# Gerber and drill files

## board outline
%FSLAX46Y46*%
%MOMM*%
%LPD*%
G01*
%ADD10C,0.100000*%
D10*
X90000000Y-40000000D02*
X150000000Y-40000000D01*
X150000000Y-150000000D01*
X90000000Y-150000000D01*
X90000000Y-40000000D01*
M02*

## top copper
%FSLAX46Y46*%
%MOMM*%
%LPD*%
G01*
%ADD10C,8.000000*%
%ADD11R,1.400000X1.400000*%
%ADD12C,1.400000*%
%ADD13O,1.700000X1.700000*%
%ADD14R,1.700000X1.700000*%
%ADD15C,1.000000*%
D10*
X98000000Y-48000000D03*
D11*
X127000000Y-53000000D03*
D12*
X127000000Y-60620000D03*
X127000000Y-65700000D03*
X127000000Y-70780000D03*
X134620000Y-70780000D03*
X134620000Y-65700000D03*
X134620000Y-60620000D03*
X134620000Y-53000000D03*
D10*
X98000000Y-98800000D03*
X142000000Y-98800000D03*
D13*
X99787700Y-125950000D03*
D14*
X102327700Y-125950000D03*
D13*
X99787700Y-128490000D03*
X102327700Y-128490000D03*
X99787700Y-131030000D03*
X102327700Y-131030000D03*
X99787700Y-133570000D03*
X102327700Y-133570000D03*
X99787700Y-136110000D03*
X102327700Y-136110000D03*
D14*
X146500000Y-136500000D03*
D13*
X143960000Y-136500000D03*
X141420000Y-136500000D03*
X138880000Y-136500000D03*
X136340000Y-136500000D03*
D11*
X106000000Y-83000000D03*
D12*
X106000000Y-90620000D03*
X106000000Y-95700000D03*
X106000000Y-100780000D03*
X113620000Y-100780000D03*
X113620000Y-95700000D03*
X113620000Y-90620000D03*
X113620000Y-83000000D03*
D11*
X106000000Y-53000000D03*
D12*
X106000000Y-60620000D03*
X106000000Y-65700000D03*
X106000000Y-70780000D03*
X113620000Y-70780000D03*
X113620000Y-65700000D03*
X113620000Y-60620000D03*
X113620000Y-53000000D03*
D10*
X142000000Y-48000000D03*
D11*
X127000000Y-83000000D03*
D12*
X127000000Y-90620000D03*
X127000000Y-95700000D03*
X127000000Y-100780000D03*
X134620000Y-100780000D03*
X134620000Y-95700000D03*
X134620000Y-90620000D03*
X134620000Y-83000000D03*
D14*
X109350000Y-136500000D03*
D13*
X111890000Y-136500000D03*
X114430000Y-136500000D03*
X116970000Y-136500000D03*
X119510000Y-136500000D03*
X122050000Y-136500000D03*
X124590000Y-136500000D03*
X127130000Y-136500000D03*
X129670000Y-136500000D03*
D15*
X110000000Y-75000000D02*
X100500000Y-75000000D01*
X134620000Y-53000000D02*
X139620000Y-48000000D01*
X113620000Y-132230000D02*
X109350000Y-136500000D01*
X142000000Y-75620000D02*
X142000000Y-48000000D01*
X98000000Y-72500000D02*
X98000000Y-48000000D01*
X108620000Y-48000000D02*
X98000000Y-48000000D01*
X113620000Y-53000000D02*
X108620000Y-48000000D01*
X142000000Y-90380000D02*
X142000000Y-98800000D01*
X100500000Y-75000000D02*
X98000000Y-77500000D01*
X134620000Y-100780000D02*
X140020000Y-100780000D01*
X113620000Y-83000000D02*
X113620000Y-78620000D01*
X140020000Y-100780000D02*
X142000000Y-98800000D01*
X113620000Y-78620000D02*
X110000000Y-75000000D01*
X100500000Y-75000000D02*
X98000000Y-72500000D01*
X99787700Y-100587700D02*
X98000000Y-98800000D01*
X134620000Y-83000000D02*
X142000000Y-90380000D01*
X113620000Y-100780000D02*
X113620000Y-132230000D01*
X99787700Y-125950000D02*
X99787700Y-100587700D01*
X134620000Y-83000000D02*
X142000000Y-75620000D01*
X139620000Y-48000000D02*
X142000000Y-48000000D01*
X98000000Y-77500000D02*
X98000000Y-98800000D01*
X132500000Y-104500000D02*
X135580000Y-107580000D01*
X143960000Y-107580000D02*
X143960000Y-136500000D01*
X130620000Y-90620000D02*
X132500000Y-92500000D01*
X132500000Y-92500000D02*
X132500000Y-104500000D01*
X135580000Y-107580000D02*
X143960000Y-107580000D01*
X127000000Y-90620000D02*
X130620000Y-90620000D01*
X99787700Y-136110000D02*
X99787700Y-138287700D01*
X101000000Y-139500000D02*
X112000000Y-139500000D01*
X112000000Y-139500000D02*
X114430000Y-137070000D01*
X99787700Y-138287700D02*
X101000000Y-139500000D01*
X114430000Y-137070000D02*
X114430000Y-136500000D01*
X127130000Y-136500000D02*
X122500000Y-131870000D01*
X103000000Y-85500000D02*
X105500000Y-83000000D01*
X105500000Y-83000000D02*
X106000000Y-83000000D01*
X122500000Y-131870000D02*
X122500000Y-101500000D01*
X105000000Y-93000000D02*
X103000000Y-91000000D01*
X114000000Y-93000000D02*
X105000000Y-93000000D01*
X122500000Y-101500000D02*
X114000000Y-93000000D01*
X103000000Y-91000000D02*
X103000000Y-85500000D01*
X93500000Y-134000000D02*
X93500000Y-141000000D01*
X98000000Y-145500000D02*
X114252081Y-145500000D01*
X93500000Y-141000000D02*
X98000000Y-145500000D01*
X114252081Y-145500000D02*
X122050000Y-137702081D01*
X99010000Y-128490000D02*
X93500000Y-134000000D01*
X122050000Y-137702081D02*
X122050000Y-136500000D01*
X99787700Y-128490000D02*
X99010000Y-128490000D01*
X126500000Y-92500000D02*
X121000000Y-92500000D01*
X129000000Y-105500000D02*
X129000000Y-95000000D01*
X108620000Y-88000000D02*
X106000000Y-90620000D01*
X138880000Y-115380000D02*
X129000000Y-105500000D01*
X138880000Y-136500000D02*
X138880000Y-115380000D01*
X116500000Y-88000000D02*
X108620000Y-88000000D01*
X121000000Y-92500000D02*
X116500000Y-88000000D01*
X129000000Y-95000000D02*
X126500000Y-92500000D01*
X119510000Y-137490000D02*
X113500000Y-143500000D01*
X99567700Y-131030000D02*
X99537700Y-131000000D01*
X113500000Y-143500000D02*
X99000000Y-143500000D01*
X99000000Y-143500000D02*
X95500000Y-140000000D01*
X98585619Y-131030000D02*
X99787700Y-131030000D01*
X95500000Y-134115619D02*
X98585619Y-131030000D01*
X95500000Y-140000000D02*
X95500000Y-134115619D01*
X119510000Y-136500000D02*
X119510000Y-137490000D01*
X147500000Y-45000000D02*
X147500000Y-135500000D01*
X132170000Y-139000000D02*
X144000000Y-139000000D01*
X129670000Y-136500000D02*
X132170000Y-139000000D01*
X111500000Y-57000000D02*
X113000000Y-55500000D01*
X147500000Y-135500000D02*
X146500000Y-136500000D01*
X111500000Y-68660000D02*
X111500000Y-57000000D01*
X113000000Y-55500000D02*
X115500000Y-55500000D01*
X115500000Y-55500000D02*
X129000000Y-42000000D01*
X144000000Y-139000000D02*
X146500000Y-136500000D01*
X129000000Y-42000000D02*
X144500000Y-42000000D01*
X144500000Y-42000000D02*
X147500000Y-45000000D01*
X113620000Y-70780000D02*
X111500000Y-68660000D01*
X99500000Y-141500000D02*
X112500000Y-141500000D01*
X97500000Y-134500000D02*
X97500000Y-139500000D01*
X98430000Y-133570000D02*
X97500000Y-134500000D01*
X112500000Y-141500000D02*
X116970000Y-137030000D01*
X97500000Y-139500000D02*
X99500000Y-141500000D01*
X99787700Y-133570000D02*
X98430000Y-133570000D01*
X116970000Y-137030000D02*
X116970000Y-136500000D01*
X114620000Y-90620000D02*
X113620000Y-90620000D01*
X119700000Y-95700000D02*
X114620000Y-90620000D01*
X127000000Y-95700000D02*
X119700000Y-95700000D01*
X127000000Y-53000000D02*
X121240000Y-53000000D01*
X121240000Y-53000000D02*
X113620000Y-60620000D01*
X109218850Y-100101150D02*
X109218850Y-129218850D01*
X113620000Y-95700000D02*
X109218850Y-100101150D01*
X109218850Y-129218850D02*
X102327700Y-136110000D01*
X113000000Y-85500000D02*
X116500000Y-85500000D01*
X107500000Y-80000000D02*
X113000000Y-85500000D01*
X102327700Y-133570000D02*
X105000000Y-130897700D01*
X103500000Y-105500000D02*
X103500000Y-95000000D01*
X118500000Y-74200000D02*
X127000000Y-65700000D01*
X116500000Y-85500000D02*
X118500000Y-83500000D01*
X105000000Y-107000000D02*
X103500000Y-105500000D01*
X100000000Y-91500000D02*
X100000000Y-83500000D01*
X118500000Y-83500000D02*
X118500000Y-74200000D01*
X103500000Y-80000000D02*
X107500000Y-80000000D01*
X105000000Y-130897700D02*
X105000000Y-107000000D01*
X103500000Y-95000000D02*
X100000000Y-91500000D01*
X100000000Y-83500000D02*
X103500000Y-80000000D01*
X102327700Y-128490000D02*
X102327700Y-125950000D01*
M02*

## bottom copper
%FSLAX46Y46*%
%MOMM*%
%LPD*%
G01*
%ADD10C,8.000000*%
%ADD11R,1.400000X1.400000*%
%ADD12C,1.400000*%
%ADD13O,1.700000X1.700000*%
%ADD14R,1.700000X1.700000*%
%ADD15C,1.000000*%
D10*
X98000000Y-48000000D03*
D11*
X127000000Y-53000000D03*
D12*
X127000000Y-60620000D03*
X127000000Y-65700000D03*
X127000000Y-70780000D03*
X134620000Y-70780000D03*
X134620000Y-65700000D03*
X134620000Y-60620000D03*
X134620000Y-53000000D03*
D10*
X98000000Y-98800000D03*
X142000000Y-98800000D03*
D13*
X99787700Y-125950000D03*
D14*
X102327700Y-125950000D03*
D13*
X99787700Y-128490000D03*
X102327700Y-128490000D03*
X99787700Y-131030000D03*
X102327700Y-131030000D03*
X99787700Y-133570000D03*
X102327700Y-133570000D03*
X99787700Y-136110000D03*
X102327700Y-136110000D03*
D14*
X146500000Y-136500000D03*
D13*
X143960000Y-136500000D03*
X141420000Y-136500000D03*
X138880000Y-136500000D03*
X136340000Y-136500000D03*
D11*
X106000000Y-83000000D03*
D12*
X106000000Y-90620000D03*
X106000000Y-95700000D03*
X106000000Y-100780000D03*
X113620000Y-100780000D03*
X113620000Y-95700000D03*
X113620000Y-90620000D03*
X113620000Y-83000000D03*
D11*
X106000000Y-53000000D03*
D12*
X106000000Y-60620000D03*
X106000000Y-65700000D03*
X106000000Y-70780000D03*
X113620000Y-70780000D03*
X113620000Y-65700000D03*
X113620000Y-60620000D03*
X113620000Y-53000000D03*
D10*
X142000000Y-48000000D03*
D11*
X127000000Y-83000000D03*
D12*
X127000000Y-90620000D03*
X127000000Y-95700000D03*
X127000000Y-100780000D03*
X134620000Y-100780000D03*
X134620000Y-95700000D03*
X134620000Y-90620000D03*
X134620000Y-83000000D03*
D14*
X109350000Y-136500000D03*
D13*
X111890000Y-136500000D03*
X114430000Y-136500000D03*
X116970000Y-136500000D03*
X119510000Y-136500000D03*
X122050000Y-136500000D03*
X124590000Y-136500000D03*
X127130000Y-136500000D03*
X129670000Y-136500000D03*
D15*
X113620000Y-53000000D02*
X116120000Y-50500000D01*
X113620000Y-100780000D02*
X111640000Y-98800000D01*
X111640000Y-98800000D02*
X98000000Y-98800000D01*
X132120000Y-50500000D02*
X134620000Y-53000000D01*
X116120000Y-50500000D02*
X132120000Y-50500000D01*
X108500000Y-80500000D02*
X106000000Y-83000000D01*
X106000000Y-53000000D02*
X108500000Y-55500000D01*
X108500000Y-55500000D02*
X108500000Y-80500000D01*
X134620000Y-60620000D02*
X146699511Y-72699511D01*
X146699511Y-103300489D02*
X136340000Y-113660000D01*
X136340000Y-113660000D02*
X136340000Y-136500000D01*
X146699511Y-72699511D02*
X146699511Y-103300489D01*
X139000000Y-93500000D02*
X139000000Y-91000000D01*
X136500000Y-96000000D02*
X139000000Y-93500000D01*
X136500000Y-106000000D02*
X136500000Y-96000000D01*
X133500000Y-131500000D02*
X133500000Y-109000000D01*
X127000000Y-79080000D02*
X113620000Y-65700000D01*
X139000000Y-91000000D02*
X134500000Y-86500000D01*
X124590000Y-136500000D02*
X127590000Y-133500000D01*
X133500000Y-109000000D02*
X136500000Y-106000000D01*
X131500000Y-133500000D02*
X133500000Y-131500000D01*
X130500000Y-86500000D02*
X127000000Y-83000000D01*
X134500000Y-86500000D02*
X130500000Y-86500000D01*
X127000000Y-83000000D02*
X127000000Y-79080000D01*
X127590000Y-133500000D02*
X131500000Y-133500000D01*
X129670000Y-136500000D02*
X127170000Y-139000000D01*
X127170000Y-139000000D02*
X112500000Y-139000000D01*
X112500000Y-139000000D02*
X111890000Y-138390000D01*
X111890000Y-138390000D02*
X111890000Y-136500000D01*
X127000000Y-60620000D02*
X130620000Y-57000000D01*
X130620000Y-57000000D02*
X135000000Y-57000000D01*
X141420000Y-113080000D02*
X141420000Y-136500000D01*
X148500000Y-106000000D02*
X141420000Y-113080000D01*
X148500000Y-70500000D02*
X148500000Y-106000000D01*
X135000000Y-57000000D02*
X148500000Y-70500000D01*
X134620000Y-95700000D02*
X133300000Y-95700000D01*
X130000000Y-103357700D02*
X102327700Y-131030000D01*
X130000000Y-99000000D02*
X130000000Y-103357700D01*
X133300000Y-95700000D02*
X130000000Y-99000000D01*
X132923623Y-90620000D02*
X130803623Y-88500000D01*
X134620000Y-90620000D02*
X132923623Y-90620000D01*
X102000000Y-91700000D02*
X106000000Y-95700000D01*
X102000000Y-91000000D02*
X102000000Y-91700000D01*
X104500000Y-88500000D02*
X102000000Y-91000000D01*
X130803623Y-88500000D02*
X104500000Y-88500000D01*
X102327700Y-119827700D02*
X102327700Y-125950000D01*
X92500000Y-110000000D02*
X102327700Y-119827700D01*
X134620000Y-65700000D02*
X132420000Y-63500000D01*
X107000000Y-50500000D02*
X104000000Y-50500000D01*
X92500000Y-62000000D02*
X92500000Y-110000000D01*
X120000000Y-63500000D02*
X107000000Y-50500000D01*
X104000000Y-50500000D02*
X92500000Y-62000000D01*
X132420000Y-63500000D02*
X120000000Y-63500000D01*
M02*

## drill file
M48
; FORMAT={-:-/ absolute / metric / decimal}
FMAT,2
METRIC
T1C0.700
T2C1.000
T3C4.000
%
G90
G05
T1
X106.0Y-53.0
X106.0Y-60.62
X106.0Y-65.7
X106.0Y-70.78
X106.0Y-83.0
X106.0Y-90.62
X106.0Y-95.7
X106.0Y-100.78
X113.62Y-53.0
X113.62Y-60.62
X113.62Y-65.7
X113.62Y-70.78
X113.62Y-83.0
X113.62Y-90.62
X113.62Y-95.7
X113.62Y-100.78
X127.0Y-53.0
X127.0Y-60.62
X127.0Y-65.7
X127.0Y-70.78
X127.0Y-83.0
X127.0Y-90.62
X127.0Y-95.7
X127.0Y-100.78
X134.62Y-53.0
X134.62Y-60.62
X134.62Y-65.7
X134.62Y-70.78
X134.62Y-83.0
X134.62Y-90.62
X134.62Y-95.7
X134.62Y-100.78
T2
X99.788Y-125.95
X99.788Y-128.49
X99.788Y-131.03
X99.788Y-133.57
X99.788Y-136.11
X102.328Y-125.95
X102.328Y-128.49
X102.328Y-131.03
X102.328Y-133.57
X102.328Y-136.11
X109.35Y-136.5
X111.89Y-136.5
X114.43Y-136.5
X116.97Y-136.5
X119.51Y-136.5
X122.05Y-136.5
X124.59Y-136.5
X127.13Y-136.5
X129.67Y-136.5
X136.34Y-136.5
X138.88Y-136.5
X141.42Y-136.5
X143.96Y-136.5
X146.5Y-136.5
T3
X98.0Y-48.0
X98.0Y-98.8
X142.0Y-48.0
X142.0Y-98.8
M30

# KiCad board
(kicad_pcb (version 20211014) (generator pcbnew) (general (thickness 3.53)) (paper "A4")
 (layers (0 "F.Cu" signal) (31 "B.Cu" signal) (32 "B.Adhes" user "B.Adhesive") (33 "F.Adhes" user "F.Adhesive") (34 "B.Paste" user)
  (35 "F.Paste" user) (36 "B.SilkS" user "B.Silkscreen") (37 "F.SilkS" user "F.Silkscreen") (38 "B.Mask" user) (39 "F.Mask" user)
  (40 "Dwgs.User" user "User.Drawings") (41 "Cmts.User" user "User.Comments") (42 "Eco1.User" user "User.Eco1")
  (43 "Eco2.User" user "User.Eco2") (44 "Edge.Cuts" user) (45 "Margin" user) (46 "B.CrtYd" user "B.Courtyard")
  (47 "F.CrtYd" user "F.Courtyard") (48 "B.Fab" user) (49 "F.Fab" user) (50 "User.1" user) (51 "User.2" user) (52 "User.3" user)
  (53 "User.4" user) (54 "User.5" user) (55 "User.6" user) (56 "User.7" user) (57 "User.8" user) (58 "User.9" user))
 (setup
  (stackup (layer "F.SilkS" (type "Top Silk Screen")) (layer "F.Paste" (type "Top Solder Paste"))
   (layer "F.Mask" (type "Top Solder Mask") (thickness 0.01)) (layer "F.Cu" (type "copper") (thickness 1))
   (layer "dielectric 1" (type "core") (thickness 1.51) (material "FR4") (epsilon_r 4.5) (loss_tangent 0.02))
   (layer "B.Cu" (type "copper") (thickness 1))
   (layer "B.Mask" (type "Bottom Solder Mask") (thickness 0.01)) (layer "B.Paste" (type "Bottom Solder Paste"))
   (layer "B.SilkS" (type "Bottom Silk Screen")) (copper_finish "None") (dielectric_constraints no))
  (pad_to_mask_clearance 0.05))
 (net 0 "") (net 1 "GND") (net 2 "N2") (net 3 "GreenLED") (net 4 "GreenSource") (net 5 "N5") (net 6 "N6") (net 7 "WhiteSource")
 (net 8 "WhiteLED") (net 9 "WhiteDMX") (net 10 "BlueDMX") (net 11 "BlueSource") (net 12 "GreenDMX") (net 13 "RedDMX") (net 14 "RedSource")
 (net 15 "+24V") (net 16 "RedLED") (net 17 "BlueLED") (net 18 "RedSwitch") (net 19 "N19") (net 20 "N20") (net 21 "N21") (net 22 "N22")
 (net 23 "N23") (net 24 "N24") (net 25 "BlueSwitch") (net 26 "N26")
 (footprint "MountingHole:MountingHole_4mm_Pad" (layer "F.Cu") (at 98 48)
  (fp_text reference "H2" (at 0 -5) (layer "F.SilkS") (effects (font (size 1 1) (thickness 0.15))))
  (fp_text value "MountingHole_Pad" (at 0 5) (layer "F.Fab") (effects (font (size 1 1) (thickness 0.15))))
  (pad "1" thru_hole circle (at 0 0) (size 8 8) (drill 4) (layers *.Cu *.Mask) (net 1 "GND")))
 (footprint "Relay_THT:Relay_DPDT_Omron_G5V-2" (layer "F.Cu") (at 127 53)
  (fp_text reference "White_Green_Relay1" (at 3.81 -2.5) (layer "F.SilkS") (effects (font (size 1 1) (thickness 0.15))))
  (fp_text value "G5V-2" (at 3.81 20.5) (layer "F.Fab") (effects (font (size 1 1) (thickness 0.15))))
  (pad "1" thru_hole rect (at 0 0) (size 1.4 1.4) (drill 0.7) (layers *.Cu *.Mask) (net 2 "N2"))
  (pad "4" thru_hole circle (at 0 7.62) (size 1.4 1.4) (drill 0.7) (layers *.Cu *.Mask) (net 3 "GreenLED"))
  (pad "6" thru_hole circle (at 0 12.7) (size 1.4 1.4) (drill 0.7) (layers *.Cu *.Mask) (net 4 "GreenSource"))
  (pad "8" thru_hole circle (at 0 17.78) (size 1.4 1.4) (drill 0.7) (layers *.Cu *.Mask) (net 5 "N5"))
  (pad "9" thru_hole circle (at 7.62 17.78) (size 1.4 1.4) (drill 0.7) (layers *.Cu *.Mask) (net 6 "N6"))
  (pad "11" thru_hole circle (at 7.62 12.7) (size 1.4 1.4) (drill 0.7) (layers *.Cu *.Mask) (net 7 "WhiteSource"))
  (pad "13" thru_hole circle (at 7.62 7.62) (size 1.4 1.4) (drill 0.7) (layers *.Cu *.Mask) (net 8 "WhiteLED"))
  (pad "16" thru_hole circle (at 7.62 0) (size 1.4 1.4) (drill 0.7) (layers *.Cu *.Mask) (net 1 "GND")))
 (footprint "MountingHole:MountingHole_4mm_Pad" (layer "F.Cu") (at 98 98.8)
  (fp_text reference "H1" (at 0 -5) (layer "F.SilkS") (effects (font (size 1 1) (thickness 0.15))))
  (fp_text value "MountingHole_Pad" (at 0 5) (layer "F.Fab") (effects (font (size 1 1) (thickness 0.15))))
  (pad "1" thru_hole circle (at 0 0) (size 8 8) (drill 4) (layers *.Cu *.Mask) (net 1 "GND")))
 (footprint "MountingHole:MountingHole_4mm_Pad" (layer "F.Cu") (at 142 98.8)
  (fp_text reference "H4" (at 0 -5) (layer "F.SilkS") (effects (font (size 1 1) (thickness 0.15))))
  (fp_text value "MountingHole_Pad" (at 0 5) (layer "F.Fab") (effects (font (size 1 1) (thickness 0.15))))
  (pad "1" thru_hole circle (at 0 0) (size 8 8) (drill 4) (layers *.Cu *.Mask) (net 1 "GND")))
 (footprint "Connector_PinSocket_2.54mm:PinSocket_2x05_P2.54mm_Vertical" (layer "F.Cu") (at 102.3277 125.95)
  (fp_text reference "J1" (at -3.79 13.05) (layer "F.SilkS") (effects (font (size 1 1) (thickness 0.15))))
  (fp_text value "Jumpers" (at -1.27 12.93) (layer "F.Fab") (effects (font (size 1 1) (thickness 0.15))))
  (pad "1a" thru_hole oval (at -2.54 0) (size 1.7 1.7) (drill 1) (layers *.Cu *.Mask) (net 1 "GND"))
  (pad "1b" thru_hole rect (at 0 0) (size 1.7 1.7) (drill 1) (layers *.Cu *.Mask) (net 7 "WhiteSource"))
  (pad "2a" thru_hole oval (at -2.54 2.54) (size 1.7 1.7) (drill 1) (layers *.Cu *.Mask) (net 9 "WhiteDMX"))
  (pad "2b" thru_hole oval (at 0 2.54) (size 1.7 1.7) (drill 1) (layers *.Cu *.Mask) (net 7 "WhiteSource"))
  (pad "3a" thru_hole oval (at -2.54 5.08) (size 1.7 1.7) (drill 1) (layers *.Cu *.Mask) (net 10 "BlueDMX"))
  (pad "3b" thru_hole oval (at 0 5.08) (size 1.7 1.7) (drill 1) (layers *.Cu *.Mask) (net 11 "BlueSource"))
  (pad "4a" thru_hole oval (at -2.54 7.62) (size 1.7 1.7) (drill 1) (layers *.Cu *.Mask) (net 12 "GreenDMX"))
  (pad "4b" thru_hole oval (at 0 7.62) (size 1.7 1.7) (drill 1) (layers *.Cu *.Mask) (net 4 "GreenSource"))
  (pad "5a" thru_hole oval (at -2.54 10.16) (size 1.7 1.7) (drill 1) (layers *.Cu *.Mask) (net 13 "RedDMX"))
  (pad "5b" thru_hole oval (at 0 10.16) (size 1.7 1.7) (drill 1) (layers *.Cu *.Mask) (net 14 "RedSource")))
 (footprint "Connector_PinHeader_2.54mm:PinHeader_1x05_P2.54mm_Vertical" (layer "F.Cu") (at 146.5 136.5 -90)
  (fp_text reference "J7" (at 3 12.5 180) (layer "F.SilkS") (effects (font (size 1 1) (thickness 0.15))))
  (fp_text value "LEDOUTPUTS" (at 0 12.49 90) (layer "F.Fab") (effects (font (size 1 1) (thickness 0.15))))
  (pad "1" thru_hole rect (at 0 0 270) (size 1.7 1.7) (drill 1) (layers *.Cu *.Mask) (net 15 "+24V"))
  (pad "2" thru_hole oval (at 0 2.54 270) (size 1.7 1.7) (drill 1) (layers *.Cu *.Mask) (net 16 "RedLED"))
  (pad "3" thru_hole oval (at 0 5.08 270) (size 1.7 1.7) (drill 1) (layers *.Cu *.Mask) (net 3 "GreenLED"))
  (pad "4" thru_hole oval (at 0 7.62 270) (size 1.7 1.7) (drill 1) (layers *.Cu *.Mask) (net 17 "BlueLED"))
  (pad "5" thru_hole oval (at 0 10.16 270) (size 1.7 1.7) (drill 1) (layers *.Cu *.Mask) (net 8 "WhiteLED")))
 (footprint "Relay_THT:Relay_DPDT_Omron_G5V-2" (layer "F.Cu") (at 106 83)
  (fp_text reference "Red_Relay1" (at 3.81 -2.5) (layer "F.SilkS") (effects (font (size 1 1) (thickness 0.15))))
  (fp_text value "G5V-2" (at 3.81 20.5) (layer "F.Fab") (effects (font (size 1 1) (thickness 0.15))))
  (pad "1" thru_hole rect (at 0 0) (size 1.4 1.4) (drill 0.7) (layers *.Cu *.Mask) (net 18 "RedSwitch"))
  (pad "4" thru_hole circle (at 0 7.62) (size 1.4 1.4) (drill 0.7) (layers *.Cu *.Mask) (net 17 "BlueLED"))
  (pad "6" thru_hole circle (at 0 12.7) (size 1.4 1.4) (drill 0.7) (layers *.Cu *.Mask) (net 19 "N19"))
  (pad "8" thru_hole circle (at 0 17.78) (size 1.4 1.4) (drill 0.7) (layers *.Cu *.Mask) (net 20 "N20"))
  (pad "9" thru_hole circle (at 7.62 17.78) (size 1.4 1.4) (drill 0.7) (layers *.Cu *.Mask) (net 1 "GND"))
  (pad "11" thru_hole circle (at 7.62 12.7) (size 1.4 1.4) (drill 0.7) (layers *.Cu *.Mask) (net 14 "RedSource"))
  (pad "13" thru_hole circle (at 7.62 7.62) (size 1.4 1.4) (drill 0.7) (layers *.Cu *.Mask) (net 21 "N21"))
  (pad "16" thru_hole circle (at 7.62 0) (size 1.4 1.4) (drill 0.7) (layers *.Cu *.Mask) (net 1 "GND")))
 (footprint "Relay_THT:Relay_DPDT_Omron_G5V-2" (layer "F.Cu") (at 106 53)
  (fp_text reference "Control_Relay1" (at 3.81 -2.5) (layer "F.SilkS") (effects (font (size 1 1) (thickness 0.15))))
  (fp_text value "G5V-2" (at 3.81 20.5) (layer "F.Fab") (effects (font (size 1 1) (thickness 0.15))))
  (pad "1" thru_hole rect (at 0 0) (size 1.4 1.4) (drill 0.7) (layers *.Cu *.Mask) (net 18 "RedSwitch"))
  (pad "4" thru_hole circle (at 0 7.62) (size 1.4 1.4) (drill 0.7) (layers *.Cu *.Mask) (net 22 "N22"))
  (pad "6" thru_hole circle (at 0 12.7) (size 1.4 1.4) (drill 0.7) (layers *.Cu *.Mask) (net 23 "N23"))
  (pad "8" thru_hole circle (at 0 17.78) (size 1.4 1.4) (drill 0.7) (layers *.Cu *.Mask) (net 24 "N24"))
  (pad "9" thru_hole circle (at 7.62 17.78) (size 1.4 1.4) (drill 0.7) (layers *.Cu *.Mask) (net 15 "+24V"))
  (pad "11" thru_hole circle (at 7.62 12.7) (size 1.4 1.4) (drill 0.7) (layers *.Cu *.Mask) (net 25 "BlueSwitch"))
  (pad "13" thru_hole circle (at 7.62 7.62) (size 1.4 1.4) (drill 0.7) (layers *.Cu *.Mask) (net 2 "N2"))
  (pad "16" thru_hole circle (at 7.62 0) (size 1.4 1.4) (drill 0.7) (layers *.Cu *.Mask) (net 1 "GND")))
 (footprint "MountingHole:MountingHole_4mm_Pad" (layer "F.Cu") (at 142 48)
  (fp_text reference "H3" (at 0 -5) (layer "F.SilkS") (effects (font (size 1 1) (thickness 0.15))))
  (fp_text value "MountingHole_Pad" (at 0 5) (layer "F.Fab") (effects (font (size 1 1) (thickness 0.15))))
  (pad "1" thru_hole circle (at 0 0) (size 8 8) (drill 4) (layers *.Cu *.Mask) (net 1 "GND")))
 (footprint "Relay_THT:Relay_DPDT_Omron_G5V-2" (layer "F.Cu") (at 127 83)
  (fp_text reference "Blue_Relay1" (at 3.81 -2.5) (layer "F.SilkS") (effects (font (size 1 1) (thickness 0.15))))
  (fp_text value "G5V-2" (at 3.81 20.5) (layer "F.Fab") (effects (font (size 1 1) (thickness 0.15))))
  (pad "1" thru_hole rect (at 0 0) (size 1.4 1.4) (drill 0.7) (layers *.Cu *.Mask) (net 25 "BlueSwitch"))
  (pad "4" thru_hole circle (at 0 7.62) (size 1.4 1.4) (drill 0.7) (layers *.Cu *.Mask) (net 16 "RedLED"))
  (pad "6" thru_hole circle (at 0 12.7) (size 1.4 1.4) (drill 0.7) (layers *.Cu *.Mask) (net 21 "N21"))
  (pad "8" thru_hole circle (at 0 17.78) (size 1.4 1.4) (drill 0.7) (layers *.Cu *.Mask) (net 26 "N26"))
  (pad "9" thru_hole circle (at 7.62 17.78) (size 1.4 1.4) (drill 0.7) (layers *.Cu *.Mask) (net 1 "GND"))
  (pad "11" thru_hole circle (at 7.62 12.7) (size 1.4 1.4) (drill 0.7) (layers *.Cu *.Mask) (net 11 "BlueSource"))
  (pad "13" thru_hole circle (at 7.62 7.62) (size 1.4 1.4) (drill 0.7) (layers *.Cu *.Mask) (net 19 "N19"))
  (pad "16" thru_hole circle (at 7.62 0) (size 1.4 1.4) (drill 0.7) (layers *.Cu *.Mask) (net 1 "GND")))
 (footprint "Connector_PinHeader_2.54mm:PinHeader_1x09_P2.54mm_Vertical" (layer "F.Cu") (at 109.35 136.5 90)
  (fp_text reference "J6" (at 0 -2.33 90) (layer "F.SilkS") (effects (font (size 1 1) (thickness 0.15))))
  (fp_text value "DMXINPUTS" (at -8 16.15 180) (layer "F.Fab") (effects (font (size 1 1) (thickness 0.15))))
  (pad "1" thru_hole rect (at 0 0 90) (size 1.7 1.7) (drill 1) (layers *.Cu *.Mask) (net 1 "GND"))
  (pad "2" thru_hole oval (at 0 2.54 90) (size 1.7 1.7) (drill 1) (layers *.Cu *.Mask) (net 15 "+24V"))
  (pad "3" thru_hole oval (at 0 5.08 90) (size 1.7 1.7) (drill 1) (layers *.Cu *.Mask) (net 13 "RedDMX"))
  (pad "4" thru_hole oval (at 0 7.62 90) (size 1.7 1.7) (drill 1) (layers *.Cu *.Mask) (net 12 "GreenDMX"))
  (pad "5" thru_hole oval (at 0 10.16 90) (size 1.7 1.7) (drill 1) (layers *.Cu *.Mask) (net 10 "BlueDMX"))
  (pad "6" thru_hole oval (at 0 12.7 90) (size 1.7 1.7) (drill 1) (layers *.Cu *.Mask) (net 9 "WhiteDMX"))
  (pad "7" thru_hole oval (at 0 15.24 90) (size 1.7 1.7) (drill 1) (layers *.Cu *.Mask) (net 25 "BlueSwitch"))
  (pad "8" thru_hole oval (at 0 17.78 90) (size 1.7 1.7) (drill 1) (layers *.Cu *.Mask) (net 18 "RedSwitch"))
  (pad "9" thru_hole oval (at 0 20.32 90) (size 1.7 1.7) (drill 1) (layers *.Cu *.Mask) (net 15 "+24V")))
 (gr_rect (start 90 40) (end 150 150) (layer "Edge.Cuts") (width 0.1) (fill none))
 (segment (start 110 75) (end 100.5 75) (width 1) (layer "F.Cu") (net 1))
 (segment (start 134.62 53) (end 139.62 48) (width 1) (layer "F.Cu") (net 1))
 (segment (start 113.62 132.23) (end 109.35 136.5) (width 1) (layer "F.Cu") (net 1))
 (segment (start 142 75.62) (end 142 48) (width 1) (layer "F.Cu") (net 1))
 (segment (start 98 72.5) (end 98 48) (width 1) (layer "F.Cu") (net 1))
 (segment (start 108.62 48) (end 98 48) (width 1) (layer "F.Cu") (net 1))
 (segment (start 113.62 53) (end 108.62 48) (width 1) (layer "F.Cu") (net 1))
 (segment (start 142 90.38) (end 142 98.8) (width 1) (layer "F.Cu") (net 1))
 (segment (start 100.5 75) (end 98 77.5) (width 1) (layer "F.Cu") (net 1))
 (segment (start 134.62 100.78) (end 140.02 100.78) (width 1) (layer "F.Cu") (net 1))
 (segment (start 113.62 83) (end 113.62 78.62) (width 1) (layer "F.Cu") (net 1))
 (segment (start 140.02 100.78) (end 142 98.8) (width 1) (layer "F.Cu") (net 1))
 (segment (start 113.62 78.62) (end 110 75) (width 1) (layer "F.Cu") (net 1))
 (segment (start 100.5 75) (end 98 72.5) (width 1) (layer "F.Cu") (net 1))
 (segment (start 99.7877 100.5877) (end 98 98.8) (width 1) (layer "F.Cu") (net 1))
 (segment (start 134.62 83) (end 142 90.38) (width 1) (layer "F.Cu") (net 1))
 (segment (start 113.62 100.78) (end 113.62 132.23) (width 1) (layer "F.Cu") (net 1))
 (segment (start 99.7877 125.95) (end 99.7877 100.5877) (width 1) (layer "F.Cu") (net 1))
 (segment (start 134.62 83) (end 142 75.62) (width 1) (layer "F.Cu") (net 1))
 (segment (start 139.62 48) (end 142 48) (width 1) (layer "F.Cu") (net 1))
 (segment (start 98 77.5) (end 98 98.8) (width 1) (layer "F.Cu") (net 1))
 (segment (start 113.62 53) (end 116.12 50.5) (width 1) (layer "B.Cu") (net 1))
 (segment (start 113.62 100.78) (end 111.64 98.8) (width 1) (layer "B.Cu") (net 1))
 (segment (start 111.64 98.8) (end 98 98.8) (width 1) (layer "B.Cu") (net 1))
 (segment (start 132.12 50.5) (end 134.62 53) (width 1) (layer "B.Cu") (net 1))
 (segment (start 116.12 50.5) (end 132.12 50.5) (width 1) (layer "B.Cu") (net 1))
 (segment (start 132.5 104.5) (end 135.58 107.58) (width 1) (layer "F.Cu") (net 16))
 (segment (start 143.96 107.58) (end 143.96 136.5) (width 1) (layer "F.Cu") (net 16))
 (segment (start 130.62 90.62) (end 132.5 92.5) (width 1) (layer "F.Cu") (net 16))
 (segment (start 132.5 92.5) (end 132.5 104.5) (width 1) (layer "F.Cu") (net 16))
 (segment (start 135.58 107.58) (end 143.96 107.58) (width 1) (layer "F.Cu") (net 16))
 (segment (start 127 90.62) (end 130.62 90.62) (width 1) (layer "F.Cu") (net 16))
 (segment (start 99.7877 136.11) (end 99.7877 138.2877) (width 1) (layer "F.Cu") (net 13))
 (segment (start 101 139.5) (end 112 139.5) (width 1) (layer "F.Cu") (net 13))
 (segment (start 112 139.5) (end 114.43 137.07) (width 1) (layer "F.Cu") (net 13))
 (segment (start 99.7877 138.2877) (end 101 139.5) (width 1) (layer "F.Cu") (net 13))
 (segment (start 114.43 137.07) (end 114.43 136.5) (width 1) (layer "F.Cu") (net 13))
 (segment (start 127.13 136.5) (end 122.5 131.87) (width 1) (layer "F.Cu") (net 18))
 (segment (start 103 85.5) (end 105.5 83) (width 1) (layer "F.Cu") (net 18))
 (segment (start 105.5 83) (end 106 83) (width 1) (layer "F.Cu") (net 18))
 (segment (start 122.5 131.87) (end 122.5 101.5) (width 1) (layer "F.Cu") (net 18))
 (segment (start 105 93) (end 103 91) (width 1) (layer "F.Cu") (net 18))
 (segment (start 114 93) (end 105 93) (width 1) (layer "F.Cu") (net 18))
 (segment (start 122.5 101.5) (end 114 93) (width 1) (layer "F.Cu") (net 18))
 (segment (start 103 91) (end 103 85.5) (width 1) (layer "F.Cu") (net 18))
 (segment (start 108.5 80.5) (end 106 83) (width 1) (layer "B.Cu") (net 18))
 (segment (start 106 53) (end 108.5 55.5) (width 1) (layer "B.Cu") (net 18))
 (segment (start 108.5 55.5) (end 108.5 80.5) (width 1) (layer "B.Cu") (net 18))
 (segment (start 134.62 60.62) (end 146.699511 72.699511) (width 1) (layer "B.Cu") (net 8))
 (segment (start 146.699511 103.300489) (end 136.34 113.66) (width 1) (layer "B.Cu") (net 8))
 (segment (start 136.34 113.66) (end 136.34 136.5) (width 1) (layer "B.Cu") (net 8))
 (segment (start 146.699511 72.699511) (end 146.699511 103.300489) (width 1) (layer "B.Cu") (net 8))
 (segment (start 93.5 134) (end 93.5 141) (width 1) (layer "F.Cu") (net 9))
 (segment (start 98 145.5) (end 114.252081 145.5) (width 1) (layer "F.Cu") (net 9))
 (segment (start 93.5 141) (end 98 145.5) (width 1) (layer "F.Cu") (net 9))
 (segment (start 114.252081 145.5) (end 122.05 137.702081) (width 1) (layer "F.Cu") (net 9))
 (segment (start 99.01 128.49) (end 93.5 134) (width 1) (layer "F.Cu") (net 9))
 (segment (start 122.05 137.702081) (end 122.05 136.5) (width 1) (layer "F.Cu") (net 9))
 (segment (start 99.7877 128.49) (end 99.01 128.49) (width 1) (layer "F.Cu") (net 9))
 (segment (start 126.5 92.5) (end 121 92.5) (width 1) (layer "F.Cu") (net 17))
 (segment (start 129 105.5) (end 129 95) (width 1) (layer "F.Cu") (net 17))
 (segment (start 108.62 88) (end 106 90.62) (width 1) (layer "F.Cu") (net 17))
 (segment (start 138.88 115.38) (end 129 105.5) (width 1) (layer "F.Cu") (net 17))
 (segment (start 138.88 136.5) (end 138.88 115.38) (width 1) (layer "F.Cu") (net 17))
 (segment (start 116.5 88) (end 108.62 88) (width 1) (layer "F.Cu") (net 17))
 (segment (start 121 92.5) (end 116.5 88) (width 1) (layer "F.Cu") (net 17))
 (segment (start 129 95) (end 126.5 92.5) (width 1) (layer "F.Cu") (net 17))
 (segment (start 119.51 137.49) (end 113.5 143.5) (width 1) (layer "F.Cu") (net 10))
 (segment (start 99.5677 131.03) (end 99.5377 131) (width 1) (layer "F.Cu") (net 10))
 (segment (start 113.5 143.5) (end 99 143.5) (width 1) (layer "F.Cu") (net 10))
 (segment (start 99 143.5) (end 95.5 140) (width 1) (layer "F.Cu") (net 10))
 (segment (start 98.585619 131.03) (end 99.7877 131.03) (width 1) (layer "F.Cu") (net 10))
 (segment (start 95.5 134.115619) (end 98.585619 131.03) (width 1) (layer "F.Cu") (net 10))
 (segment (start 95.5 140) (end 95.5 134.115619) (width 1) (layer "F.Cu") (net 10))
 (segment (start 119.51 136.5) (end 119.51 137.49) (width 1) (layer "F.Cu") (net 10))
 (segment (start 139 93.5) (end 139 91) (width 1) (layer "B.Cu") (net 25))
 (segment (start 136.5 96) (end 139 93.5) (width 1) (layer "B.Cu") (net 25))
 (segment (start 136.5 106) (end 136.5 96) (width 1) (layer "B.Cu") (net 25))
 (segment (start 133.5 131.5) (end 133.5 109) (width 1) (layer "B.Cu") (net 25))
 (segment (start 127 79.08) (end 113.62 65.7) (width 1) (layer "B.Cu") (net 25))
 (segment (start 139 91) (end 134.5 86.5) (width 1) (layer "B.Cu") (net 25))
 (segment (start 124.59 136.5) (end 127.59 133.5) (width 1) (layer "B.Cu") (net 25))
 (segment (start 133.5 109) (end 136.5 106) (width 1) (layer "B.Cu") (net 25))
 (segment (start 131.5 133.5) (end 133.5 131.5) (width 1) (layer "B.Cu") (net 25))
 (segment (start 130.5 86.5) (end 127 83) (width 1) (layer "B.Cu") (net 25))
 (segment (start 134.5 86.5) (end 130.5 86.5) (width 1) (layer "B.Cu") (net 25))
 (segment (start 127 83) (end 127 79.08) (width 1) (layer "B.Cu") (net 25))
 (segment (start 127.59 133.5) (end 131.5 133.5) (width 1) (layer "B.Cu") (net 25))
 (segment (start 147.5 45) (end 147.5 135.5) (width 1) (layer "F.Cu") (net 15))
 (segment (start 132.17 139) (end 144 139) (width 1) (layer "F.Cu") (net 15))
 (segment (start 129.67 136.5) (end 132.17 139) (width 1) (layer "F.Cu") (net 15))
 (segment (start 111.5 57) (end 113 55.5) (width 1) (layer "F.Cu") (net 15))
 (segment (start 147.5 135.5) (end 146.5 136.5) (width 1) (layer "F.Cu") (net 15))
 (segment (start 111.5 68.66) (end 111.5 57) (width 1) (layer "F.Cu") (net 15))
 (segment (start 113 55.5) (end 115.5 55.5) (width 1) (layer "F.Cu") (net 15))
 (segment (start 115.5 55.5) (end 129 42) (width 1) (layer "F.Cu") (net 15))
 (segment (start 144 139) (end 146.5 136.5) (width 1) (layer "F.Cu") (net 15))
 (segment (start 129 42) (end 144.5 42) (width 1) (layer "F.Cu") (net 15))
 (segment (start 144.5 42) (end 147.5 45) (width 1) (layer "F.Cu") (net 15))
 (segment (start 113.62 70.78) (end 111.5 68.66) (width 1) (layer "F.Cu") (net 15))
 (segment (start 129.67 136.5) (end 127.17 139) (width 1) (layer "B.Cu") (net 15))
 (segment (start 127.17 139) (end 112.5 139) (width 1) (layer "B.Cu") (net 15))
 (segment (start 112.5 139) (end 111.89 138.39) (width 1) (layer "B.Cu") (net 15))
 (segment (start 111.89 138.39) (end 111.89 136.5) (width 1) (layer "B.Cu") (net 15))
 (segment (start 99.5 141.5) (end 112.5 141.5) (width 1) (layer "F.Cu") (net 12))
 (segment (start 97.5 134.5) (end 97.5 139.5) (width 1) (layer "F.Cu") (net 12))
 (segment (start 98.43 133.57) (end 97.5 134.5) (width 1) (layer "F.Cu") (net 12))
 (segment (start 112.5 141.5) (end 116.97 137.03) (width 1) (layer "F.Cu") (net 12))
 (segment (start 97.5 139.5) (end 99.5 141.5) (width 1) (layer "F.Cu") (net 12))
 (segment (start 99.7877 133.57) (end 98.43 133.57) (width 1) (layer "F.Cu") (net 12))
 (segment (start 116.97 137.03) (end 116.97 136.5) (width 1) (layer "F.Cu") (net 12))
 (segment (start 127 60.62) (end 130.62 57) (width 1) (layer "B.Cu") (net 3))
 (segment (start 130.62 57) (end 135 57) (width 1) (layer "B.Cu") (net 3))
 (segment (start 141.42 113.08) (end 141.42 136.5) (width 1) (layer "B.Cu") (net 3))
 (segment (start 148.5 106) (end 141.42 113.08) (width 1) (layer "B.Cu") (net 3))
 (segment (start 148.5 70.5) (end 148.5 106) (width 1) (layer "B.Cu") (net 3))
 (segment (start 135 57) (end 148.5 70.5) (width 1) (layer "B.Cu") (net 3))
 (segment (start 114.62 90.62) (end 113.62 90.62) (width 1) (layer "F.Cu") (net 21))
 (segment (start 119.7 95.7) (end 114.62 90.62) (width 1) (layer "F.Cu") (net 21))
 (segment (start 127 95.7) (end 119.7 95.7) (width 1) (layer "F.Cu") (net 21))
 (segment (start 134.62 95.7) (end 133.3 95.7) (width 1) (layer "B.Cu") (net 11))
 (segment (start 130 103.3577) (end 102.3277 131.03) (width 1) (layer "B.Cu") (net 11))
 (segment (start 130 99) (end 130 103.3577) (width 1) (layer "B.Cu") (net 11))
 (segment (start 133.3 95.7) (end 130 99) (width 1) (layer "B.Cu") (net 11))
 (segment (start 132.923623 90.62) (end 130.803623 88.5) (width 1) (layer "B.Cu") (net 19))
 (segment (start 134.62 90.62) (end 132.923623 90.62) (width 1) (layer "B.Cu") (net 19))
 (segment (start 102 91.7) (end 106 95.7) (width 1) (layer "B.Cu") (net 19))
 (segment (start 102 91) (end 102 91.7) (width 1) (layer "B.Cu") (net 19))
 (segment (start 104.5 88.5) (end 102 91) (width 1) (layer "B.Cu") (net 19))
 (segment (start 130.803623 88.5) (end 104.5 88.5) (width 1) (layer "B.Cu") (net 19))
 (segment (start 127 53) (end 121.24 53) (width 1) (layer "F.Cu") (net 2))
 (segment (start 121.24 53) (end 113.62 60.62) (width 1) (layer "F.Cu") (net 2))
 (segment (start 109.21885 100.10115) (end 109.21885 129.21885) (width 1) (layer "F.Cu") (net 14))
 (segment (start 113.62 95.7) (end 109.21885 100.10115) (width 1) (layer "F.Cu") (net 14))
 (segment (start 109.21885 129.21885) (end 102.3277 136.11) (width 1) (layer "F.Cu") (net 14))
 (segment (start 113 85.5) (end 116.5 85.5) (width 1) (layer "F.Cu") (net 4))
 (segment (start 107.5 80) (end 113 85.5) (width 1) (layer "F.Cu") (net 4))
 (segment (start 102.3277 133.57) (end 105 130.8977) (width 1) (layer "F.Cu") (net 4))
 (segment (start 103.5 105.5) (end 103.5 95) (width 1) (layer "F.Cu") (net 4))
 (segment (start 118.5 74.2) (end 127 65.7) (width 1) (layer "F.Cu") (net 4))
 (segment (start 116.5 85.5) (end 118.5 83.5) (width 1) (layer "F.Cu") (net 4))
 (segment (start 105 107) (end 103.5 105.5) (width 1) (layer "F.Cu") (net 4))
 (segment (start 100 91.5) (end 100 83.5) (width 1) (layer "F.Cu") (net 4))
 (segment (start 118.5 83.5) (end 118.5 74.2) (width 1) (layer "F.Cu") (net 4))
 (segment (start 103.5 80) (end 107.5 80) (width 1) (layer "F.Cu") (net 4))
 (segment (start 105 130.8977) (end 105 107) (width 1) (layer "F.Cu") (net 4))
 (segment (start 103.5 95) (end 100 91.5) (width 1) (layer "F.Cu") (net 4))
 (segment (start 100 83.5) (end 103.5 80) (width 1) (layer "F.Cu") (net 4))
 (segment (start 102.3277 128.49) (end 102.3277 125.95) (width 1) (layer "F.Cu") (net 7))
 (segment (start 102.3277 119.8277) (end 102.3277 125.95) (width 1) (layer "B.Cu") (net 7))
 (segment (start 92.5 110) (end 102.3277 119.8277) (width 1) (layer "B.Cu") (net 7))
 (segment (start 134.62 65.7) (end 132.42 63.5) (width 1) (layer "B.Cu") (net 7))
 (segment (start 107 50.5) (end 104 50.5) (width 1) (layer "B.Cu") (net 7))
 (segment (start 92.5 62) (end 92.5 110) (width 1) (layer "B.Cu") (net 7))
 (segment (start 120 63.5) (end 107 50.5) (width 1) (layer "B.Cu") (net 7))
 (segment (start 104 50.5) (end 92.5 62) (width 1) (layer "B.Cu") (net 7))
 (segment (start 132.42 63.5) (end 120 63.5) (width 1) (layer "B.Cu") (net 7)))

